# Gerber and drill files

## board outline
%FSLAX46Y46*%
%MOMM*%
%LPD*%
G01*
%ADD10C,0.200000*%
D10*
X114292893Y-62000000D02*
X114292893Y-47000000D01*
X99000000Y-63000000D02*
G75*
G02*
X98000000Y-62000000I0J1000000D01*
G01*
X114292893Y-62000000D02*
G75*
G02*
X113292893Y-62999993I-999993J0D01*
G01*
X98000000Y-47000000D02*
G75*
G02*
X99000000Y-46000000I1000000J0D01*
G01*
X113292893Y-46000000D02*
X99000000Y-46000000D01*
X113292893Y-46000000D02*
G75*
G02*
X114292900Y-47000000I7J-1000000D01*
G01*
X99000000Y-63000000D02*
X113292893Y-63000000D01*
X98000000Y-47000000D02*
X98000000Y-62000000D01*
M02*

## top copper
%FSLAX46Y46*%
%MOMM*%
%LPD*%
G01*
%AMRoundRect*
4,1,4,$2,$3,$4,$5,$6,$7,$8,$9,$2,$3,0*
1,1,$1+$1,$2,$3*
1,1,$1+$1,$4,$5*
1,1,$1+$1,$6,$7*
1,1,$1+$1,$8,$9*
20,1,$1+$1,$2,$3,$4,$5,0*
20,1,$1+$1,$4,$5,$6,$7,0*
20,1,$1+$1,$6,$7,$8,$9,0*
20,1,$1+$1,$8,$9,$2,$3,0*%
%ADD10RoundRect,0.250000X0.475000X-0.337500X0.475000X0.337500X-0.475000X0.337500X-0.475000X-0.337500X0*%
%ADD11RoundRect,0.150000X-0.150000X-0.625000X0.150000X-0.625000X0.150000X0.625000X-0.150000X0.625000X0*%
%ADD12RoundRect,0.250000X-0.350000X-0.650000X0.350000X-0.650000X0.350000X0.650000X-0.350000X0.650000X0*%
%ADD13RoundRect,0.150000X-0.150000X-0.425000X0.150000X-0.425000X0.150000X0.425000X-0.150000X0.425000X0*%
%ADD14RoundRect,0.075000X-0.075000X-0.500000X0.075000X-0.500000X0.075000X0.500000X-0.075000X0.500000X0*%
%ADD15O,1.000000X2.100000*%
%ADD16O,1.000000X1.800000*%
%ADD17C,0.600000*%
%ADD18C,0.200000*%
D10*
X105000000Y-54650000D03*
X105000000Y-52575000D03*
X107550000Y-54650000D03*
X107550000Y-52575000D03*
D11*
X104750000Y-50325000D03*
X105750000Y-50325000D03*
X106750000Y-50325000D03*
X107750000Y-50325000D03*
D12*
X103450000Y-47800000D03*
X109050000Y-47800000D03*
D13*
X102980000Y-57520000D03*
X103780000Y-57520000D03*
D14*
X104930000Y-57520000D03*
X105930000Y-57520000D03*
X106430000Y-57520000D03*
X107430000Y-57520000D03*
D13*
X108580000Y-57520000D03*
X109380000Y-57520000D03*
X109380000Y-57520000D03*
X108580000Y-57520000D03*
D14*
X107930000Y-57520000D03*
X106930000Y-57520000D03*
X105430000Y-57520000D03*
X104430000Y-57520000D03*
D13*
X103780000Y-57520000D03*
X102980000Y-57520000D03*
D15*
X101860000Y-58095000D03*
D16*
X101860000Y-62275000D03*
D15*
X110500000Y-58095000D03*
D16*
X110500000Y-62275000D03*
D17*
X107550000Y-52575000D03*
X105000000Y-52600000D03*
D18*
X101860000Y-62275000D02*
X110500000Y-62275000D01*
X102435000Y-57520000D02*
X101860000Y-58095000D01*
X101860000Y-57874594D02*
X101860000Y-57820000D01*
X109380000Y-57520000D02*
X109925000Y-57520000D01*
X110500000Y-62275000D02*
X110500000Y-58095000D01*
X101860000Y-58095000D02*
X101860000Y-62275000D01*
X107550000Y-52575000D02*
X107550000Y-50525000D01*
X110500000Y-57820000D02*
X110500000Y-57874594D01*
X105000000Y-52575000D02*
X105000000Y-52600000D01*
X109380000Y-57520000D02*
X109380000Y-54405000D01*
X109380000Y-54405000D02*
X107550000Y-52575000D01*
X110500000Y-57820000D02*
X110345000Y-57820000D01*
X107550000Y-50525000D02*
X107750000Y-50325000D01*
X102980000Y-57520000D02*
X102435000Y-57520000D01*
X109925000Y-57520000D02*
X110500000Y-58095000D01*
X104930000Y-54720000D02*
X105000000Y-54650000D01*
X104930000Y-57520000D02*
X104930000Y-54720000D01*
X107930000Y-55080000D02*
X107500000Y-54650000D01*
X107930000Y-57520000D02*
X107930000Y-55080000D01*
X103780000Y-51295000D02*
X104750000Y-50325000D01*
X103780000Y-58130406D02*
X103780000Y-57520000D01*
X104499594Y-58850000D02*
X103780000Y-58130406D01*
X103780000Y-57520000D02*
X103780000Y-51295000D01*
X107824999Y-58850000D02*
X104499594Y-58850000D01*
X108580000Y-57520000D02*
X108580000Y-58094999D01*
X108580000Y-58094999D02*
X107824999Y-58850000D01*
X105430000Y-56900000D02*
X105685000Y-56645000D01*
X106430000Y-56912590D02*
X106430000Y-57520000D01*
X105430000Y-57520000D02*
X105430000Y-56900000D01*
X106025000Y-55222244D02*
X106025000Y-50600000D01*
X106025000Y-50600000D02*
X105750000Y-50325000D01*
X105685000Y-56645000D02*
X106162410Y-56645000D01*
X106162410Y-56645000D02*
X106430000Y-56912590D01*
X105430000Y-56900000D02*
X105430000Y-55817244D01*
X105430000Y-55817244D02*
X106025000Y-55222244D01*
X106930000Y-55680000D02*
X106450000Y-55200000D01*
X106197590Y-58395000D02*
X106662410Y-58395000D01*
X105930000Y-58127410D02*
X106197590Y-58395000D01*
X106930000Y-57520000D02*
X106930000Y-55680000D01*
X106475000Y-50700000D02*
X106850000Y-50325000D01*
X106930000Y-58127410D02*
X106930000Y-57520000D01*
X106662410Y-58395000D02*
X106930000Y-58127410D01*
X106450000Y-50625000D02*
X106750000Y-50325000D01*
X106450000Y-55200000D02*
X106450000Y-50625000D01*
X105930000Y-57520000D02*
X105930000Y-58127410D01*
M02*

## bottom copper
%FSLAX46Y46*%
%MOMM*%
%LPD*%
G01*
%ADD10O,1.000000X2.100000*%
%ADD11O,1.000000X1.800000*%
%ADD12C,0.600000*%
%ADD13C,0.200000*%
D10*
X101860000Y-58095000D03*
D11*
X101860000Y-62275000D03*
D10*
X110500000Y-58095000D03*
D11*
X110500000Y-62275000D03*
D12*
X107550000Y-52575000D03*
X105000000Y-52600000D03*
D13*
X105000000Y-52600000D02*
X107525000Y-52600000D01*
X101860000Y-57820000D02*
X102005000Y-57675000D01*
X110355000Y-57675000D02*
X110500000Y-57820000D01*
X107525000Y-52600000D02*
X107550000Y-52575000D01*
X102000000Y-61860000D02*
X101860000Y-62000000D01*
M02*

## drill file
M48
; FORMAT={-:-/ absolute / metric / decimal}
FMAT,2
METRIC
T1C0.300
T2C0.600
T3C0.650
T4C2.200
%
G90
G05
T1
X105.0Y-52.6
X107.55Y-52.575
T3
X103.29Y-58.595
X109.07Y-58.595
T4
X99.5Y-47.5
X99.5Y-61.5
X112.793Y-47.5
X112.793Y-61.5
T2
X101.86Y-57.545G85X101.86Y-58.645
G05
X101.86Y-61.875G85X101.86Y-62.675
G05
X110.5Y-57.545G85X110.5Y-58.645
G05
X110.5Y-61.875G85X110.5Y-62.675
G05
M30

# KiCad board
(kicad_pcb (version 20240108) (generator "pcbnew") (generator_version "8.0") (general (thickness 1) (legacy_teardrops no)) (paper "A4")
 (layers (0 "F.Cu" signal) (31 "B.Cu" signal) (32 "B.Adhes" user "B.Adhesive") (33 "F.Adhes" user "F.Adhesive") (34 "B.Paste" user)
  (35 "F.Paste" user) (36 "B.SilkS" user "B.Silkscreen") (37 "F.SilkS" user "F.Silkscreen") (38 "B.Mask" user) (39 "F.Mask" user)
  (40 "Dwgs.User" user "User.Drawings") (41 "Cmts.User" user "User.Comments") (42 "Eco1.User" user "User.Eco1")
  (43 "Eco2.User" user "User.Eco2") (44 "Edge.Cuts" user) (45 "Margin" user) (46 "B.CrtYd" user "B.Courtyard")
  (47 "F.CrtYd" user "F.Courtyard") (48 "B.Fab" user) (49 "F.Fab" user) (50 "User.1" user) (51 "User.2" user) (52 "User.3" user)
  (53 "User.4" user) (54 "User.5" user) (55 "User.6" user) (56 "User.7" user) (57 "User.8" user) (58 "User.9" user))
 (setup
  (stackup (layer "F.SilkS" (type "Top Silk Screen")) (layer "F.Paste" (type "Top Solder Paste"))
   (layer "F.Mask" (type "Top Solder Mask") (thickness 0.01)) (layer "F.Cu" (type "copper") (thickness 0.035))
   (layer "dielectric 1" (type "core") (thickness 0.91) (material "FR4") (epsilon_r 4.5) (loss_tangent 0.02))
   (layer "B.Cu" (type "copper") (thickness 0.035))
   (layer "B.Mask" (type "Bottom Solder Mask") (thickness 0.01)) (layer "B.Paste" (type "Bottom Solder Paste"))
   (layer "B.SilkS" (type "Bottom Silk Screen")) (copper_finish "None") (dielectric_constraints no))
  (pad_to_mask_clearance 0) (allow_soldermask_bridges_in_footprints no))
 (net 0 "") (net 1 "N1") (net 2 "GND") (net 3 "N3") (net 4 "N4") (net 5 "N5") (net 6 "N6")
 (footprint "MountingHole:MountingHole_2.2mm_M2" (layer "F.Cu") (at 112.792893 47.5)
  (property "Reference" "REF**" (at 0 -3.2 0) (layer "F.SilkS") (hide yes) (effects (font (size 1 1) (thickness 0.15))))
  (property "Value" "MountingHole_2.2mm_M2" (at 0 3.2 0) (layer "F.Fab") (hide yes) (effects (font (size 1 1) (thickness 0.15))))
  (pad "" np_thru_hole circle (at 0 0) (size 2.2 2.2) (drill 2.2) (layers "*.Cu" "*.Mask")))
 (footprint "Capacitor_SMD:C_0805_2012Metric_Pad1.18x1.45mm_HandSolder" (layer "F.Cu") (at 105 53.6125 90)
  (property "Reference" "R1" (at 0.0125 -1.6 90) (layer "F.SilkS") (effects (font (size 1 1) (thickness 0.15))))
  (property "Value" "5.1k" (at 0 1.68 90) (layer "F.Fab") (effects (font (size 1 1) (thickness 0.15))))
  (pad "1" smd roundrect (at -1.0375 0 90) (size 1.175 1.45) (layers "F.Cu" "F.Paste" "F.Mask") (roundrect_rratio 0.212766) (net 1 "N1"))
  (pad "2" smd roundrect (at 1.0375 0 90) (size 1.175 1.45) (layers "F.Cu" "F.Paste" "F.Mask") (roundrect_rratio 0.212766) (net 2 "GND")))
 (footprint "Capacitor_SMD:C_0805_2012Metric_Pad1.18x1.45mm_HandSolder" (layer "F.Cu") (at 107.55 53.6125 90)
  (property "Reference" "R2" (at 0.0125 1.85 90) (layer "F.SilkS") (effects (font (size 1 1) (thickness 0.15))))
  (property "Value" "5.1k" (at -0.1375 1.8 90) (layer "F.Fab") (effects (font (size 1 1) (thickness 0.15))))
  (pad "1" smd roundrect (at -1.0375 0 90) (size 1.175 1.45) (layers "F.Cu" "F.Paste" "F.Mask") (roundrect_rratio 0.212766) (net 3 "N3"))
  (pad "2" smd roundrect (at 1.0375 0 90) (size 1.175 1.45) (layers "F.Cu" "F.Paste" "F.Mask") (roundrect_rratio 0.212766) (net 2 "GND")))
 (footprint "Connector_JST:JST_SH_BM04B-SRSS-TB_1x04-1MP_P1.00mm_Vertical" (layer "F.Cu") (at 106.25 49)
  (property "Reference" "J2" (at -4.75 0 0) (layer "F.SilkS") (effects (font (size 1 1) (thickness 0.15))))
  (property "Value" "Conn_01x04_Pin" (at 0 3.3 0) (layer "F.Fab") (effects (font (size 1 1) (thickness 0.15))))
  (pad "1" smd roundrect (at -1.5 1.325) (size 0.6 1.55) (layers "F.Cu" "F.Paste" "F.Mask") (roundrect_rratio 0.25) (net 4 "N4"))
  (pad "2" smd roundrect (at -0.5 1.325) (size 0.6 1.55) (layers "F.Cu" "F.Paste" "F.Mask") (roundrect_rratio 0.25) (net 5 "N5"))
  (pad "3" smd roundrect (at 0.5 1.325) (size 0.6 1.55) (layers "F.Cu" "F.Paste" "F.Mask") (roundrect_rratio 0.25) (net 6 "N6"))
  (pad "4" smd roundrect (at 1.5 1.325) (size 0.6 1.55) (layers "F.Cu" "F.Paste" "F.Mask") (roundrect_rratio 0.25) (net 2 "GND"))
  (pad "MP" smd roundrect (at -2.8 -1.2) (size 1.2 1.8) (layers "F.Cu" "F.Paste" "F.Mask") (roundrect_rratio 0.208333))
  (pad "MP" smd roundrect (at 2.8 -1.2) (size 1.2 1.8) (layers "F.Cu" "F.Paste" "F.Mask") (roundrect_rratio 0.208333)))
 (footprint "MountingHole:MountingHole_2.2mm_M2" (layer "F.Cu") (at 112.792893 61.5)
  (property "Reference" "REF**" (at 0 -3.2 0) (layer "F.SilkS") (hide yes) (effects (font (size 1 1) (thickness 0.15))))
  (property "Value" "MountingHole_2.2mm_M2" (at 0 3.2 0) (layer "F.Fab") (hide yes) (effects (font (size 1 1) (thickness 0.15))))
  (pad "" np_thru_hole circle (at 0 0) (size 2.2 2.2) (drill 2.2) (layers "*.Cu" "*.Mask")))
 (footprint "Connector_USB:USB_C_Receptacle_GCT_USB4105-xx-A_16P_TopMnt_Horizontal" (layer "F.Cu") (at 106.18 61.2)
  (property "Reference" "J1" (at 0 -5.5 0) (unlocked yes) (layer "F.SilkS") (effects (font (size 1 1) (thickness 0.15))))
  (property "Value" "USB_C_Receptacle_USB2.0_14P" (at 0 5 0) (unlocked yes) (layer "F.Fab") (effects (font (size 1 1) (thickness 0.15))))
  (pad "" np_thru_hole circle (at -2.89 -2.605) (size 0.65 0.65) (drill 0.65) (layers "F&B.Cu" "*.Mask"))
  (pad "" np_thru_hole circle (at 2.89 -2.605) (size 0.65 0.65) (drill 0.65) (layers "F&B.Cu" "*.Mask"))
  (pad "A1" smd roundrect (at -3.2 -3.68) (size 0.6 1.15) (layers "F.Cu" "F.Paste" "F.Mask") (roundrect_rratio 0.25) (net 2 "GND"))
  (pad "A4" smd roundrect (at -2.4 -3.68) (size 0.6 1.15) (layers "F.Cu" "F.Paste" "F.Mask") (roundrect_rratio 0.25) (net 4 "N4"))
  (pad "A5" smd roundrect (at -1.25 -3.68) (size 0.3 1.15) (layers "F.Cu" "F.Paste" "F.Mask") (roundrect_rratio 0.25) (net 1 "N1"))
  (pad "A6" smd roundrect (at -0.25 -3.68) (size 0.3 1.15) (layers "F.Cu" "F.Paste" "F.Mask") (roundrect_rratio 0.25) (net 6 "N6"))
  (pad "A7" smd roundrect (at 0.25 -3.68) (size 0.3 1.15) (layers "F.Cu" "F.Paste" "F.Mask") (roundrect_rratio 0.25) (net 5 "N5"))
  (pad "A8" smd roundrect (at 1.25 -3.68) (size 0.3 1.15) (layers "F.Cu" "F.Paste" "F.Mask") (roundrect_rratio 0.25))
  (pad "A9" smd roundrect (at 2.4 -3.68) (size 0.6 1.15) (layers "F.Cu" "F.Paste" "F.Mask") (roundrect_rratio 0.25) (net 4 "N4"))
  (pad "A12" smd roundrect (at 3.2 -3.68) (size 0.6 1.15) (layers "F.Cu" "F.Paste" "F.Mask") (roundrect_rratio 0.25) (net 2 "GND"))
  (pad "B1" smd roundrect (at 3.2 -3.68) (size 0.6 1.15) (layers "F.Cu" "F.Paste" "F.Mask") (roundrect_rratio 0.25) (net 2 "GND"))
  (pad "B4" smd roundrect (at 2.4 -3.68) (size 0.6 1.15) (layers "F.Cu" "F.Paste" "F.Mask") (roundrect_rratio 0.25) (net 4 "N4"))
  (pad "B5" smd roundrect (at 1.75 -3.68) (size 0.3 1.15) (layers "F.Cu" "F.Paste" "F.Mask") (roundrect_rratio 0.25) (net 3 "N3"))
  (pad "B6" smd roundrect (at 0.75 -3.68) (size 0.3 1.15) (layers "F.Cu" "F.Paste" "F.Mask") (roundrect_rratio 0.25) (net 6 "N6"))
  (pad "B7" smd roundrect (at -0.75 -3.68) (size 0.3 1.15) (layers "F.Cu" "F.Paste" "F.Mask") (roundrect_rratio 0.25) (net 5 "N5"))
  (pad "B8" smd roundrect (at -1.75 -3.68) (size 0.3 1.15) (layers "F.Cu" "F.Paste" "F.Mask") (roundrect_rratio 0.25))
  (pad "B9" smd roundrect (at -2.4 -3.68) (size 0.6 1.15) (layers "F.Cu" "F.Paste" "F.Mask") (roundrect_rratio 0.25) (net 4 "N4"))
  (pad "B12" smd roundrect (at -3.2 -3.68) (size 0.6 1.15) (layers "F.Cu" "F.Paste" "F.Mask") (roundrect_rratio 0.25) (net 2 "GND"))
  (pad "S1" thru_hole oval (at -4.32 -3.105) (size 1 2.1) (drill oval 0.6 1.7) (layers "*.Cu" "*.Mask" "F.Paste") (remove_unused_layers no)
   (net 2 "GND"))
  (pad "S1" thru_hole oval (at -4.32 1.075) (size 1 1.8) (drill oval 0.6 1.4) (layers "*.Cu" "*.Mask" "F.Paste") (remove_unused_layers no)
   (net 2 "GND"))
  (pad "S1" thru_hole oval (at 4.32 -3.105) (size 1 2.1) (drill oval 0.6 1.7) (layers "*.Cu" "*.Mask" "F.Paste") (remove_unused_layers no)
   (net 2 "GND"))
  (pad "S1" thru_hole oval (at 4.32 1.075) (size 1 1.8) (drill oval 0.6 1.4) (layers "*.Cu" "*.Mask" "F.Paste") (remove_unused_layers no)
   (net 2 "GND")))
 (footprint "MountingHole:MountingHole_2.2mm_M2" (layer "F.Cu") (at 99.5 61.5)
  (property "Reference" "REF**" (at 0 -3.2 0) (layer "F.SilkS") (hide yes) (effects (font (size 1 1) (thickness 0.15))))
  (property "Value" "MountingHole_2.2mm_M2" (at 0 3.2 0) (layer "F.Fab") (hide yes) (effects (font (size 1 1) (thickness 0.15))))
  (pad "" np_thru_hole circle (at 0 0) (size 2.2 2.2) (drill 2.2) (layers "*.Cu" "*.Mask")))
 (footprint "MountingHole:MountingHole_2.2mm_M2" (layer "F.Cu") (at 99.5 47.5)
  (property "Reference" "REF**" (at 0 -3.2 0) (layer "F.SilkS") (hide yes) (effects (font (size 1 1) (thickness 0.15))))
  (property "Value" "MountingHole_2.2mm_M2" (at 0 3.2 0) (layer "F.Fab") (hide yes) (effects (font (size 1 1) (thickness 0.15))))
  (pad "" np_thru_hole circle (at 0 0) (size 2.2 2.2) (drill 2.2) (layers "*.Cu" "*.Mask")))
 (gr_line (start 114.292893 62) (end 114.292893 47) (stroke (width 0.2) (type default)) (layer "Edge.Cuts"))
 (gr_arc (start 99 63) (mid 98.292896 62.707106) (end 98 62) (stroke (width 0.2) (type default)) (layer "Edge.Cuts"))
 (gr_arc (start 114.292893 62) (mid 114 62.707107) (end 113.292893 63) (stroke (width 0.2) (type default)) (layer "Edge.Cuts"))
 (gr_arc (start 98 47) (mid 98.292893 46.292893) (end 99 46) (stroke (width 0.2) (type default)) (layer "Edge.Cuts"))
 (gr_line (start 113.292893 46) (end 99 46) (stroke (width 0.2) (type default)) (layer "Edge.Cuts"))
 (gr_arc (start 113.292893 46) (mid 114 46.292893) (end 114.292893 47) (stroke (width 0.2) (type default)) (layer "Edge.Cuts"))
 (gr_line (start 99 63) (end 113.292893 63) (stroke (width 0.2) (type default)) (layer "Edge.Cuts"))
 (gr_line (start 98 47) (end 98 62) (stroke (width 0.2) (type default)) (layer "Edge.Cuts"))
 (segment (start 101.86 62.275) (end 110.5 62.275) (width 0.2) (layer "F.Cu") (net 2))
 (segment (start 102.435 57.52) (end 101.86 58.095) (width 0.2) (layer "F.Cu") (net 2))
 (segment (start 101.86 57.874594) (end 101.86 57.82) (width 0.2) (layer "F.Cu") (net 2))
 (segment (start 109.38 57.52) (end 109.925 57.52) (width 0.2) (layer "F.Cu") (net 2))
 (segment (start 110.5 62.275) (end 110.5 58.095) (width 0.2) (layer "F.Cu") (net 2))
 (segment (start 101.86 58.095) (end 101.86 62.275) (width 0.2) (layer "F.Cu") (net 2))
 (segment (start 107.55 52.575) (end 107.55 50.525) (width 0.2) (layer "F.Cu") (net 2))
 (segment (start 110.5 57.82) (end 110.5 57.874594) (width 0.2) (layer "F.Cu") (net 2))
 (segment (start 105 52.575) (end 105 52.6) (width 0.2) (layer "F.Cu") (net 2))
 (segment (start 109.38 57.52) (end 109.38 54.405) (width 0.2) (layer "F.Cu") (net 2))
 (segment (start 109.38 54.405) (end 107.55 52.575) (width 0.2) (layer "F.Cu") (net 2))
 (segment (start 110.5 57.82) (end 110.345 57.82) (width 0.2) (layer "F.Cu") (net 2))
 (segment (start 107.55 50.525) (end 107.75 50.325) (width 0.2) (layer "F.Cu") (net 2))
 (segment (start 102.98 57.52) (end 102.435 57.52) (width 0.2) (layer "F.Cu") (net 2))
 (segment (start 109.925 57.52) (end 110.5 58.095) (width 0.2) (layer "F.Cu") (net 2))
 (via (at 107.55 52.575) (size 0.6) (drill 0.3) (layers "F.Cu" "B.Cu") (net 2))
 (via (at 105 52.6) (size 0.6) (drill 0.3) (layers "F.Cu" "B.Cu") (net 2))
 (segment (start 105 52.6) (end 107.525 52.6) (width 0.2) (layer "B.Cu") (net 2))
 (segment (start 101.86 57.82) (end 102.005 57.675) (width 0.2) (layer "B.Cu") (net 2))
 (segment (start 110.355 57.675) (end 110.5 57.82) (width 0.2) (layer "B.Cu") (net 2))
 (segment (start 107.525 52.6) (end 107.55 52.575) (width 0.2) (layer "B.Cu") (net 2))
 (segment (start 102 61.86) (end 101.86 62) (width 0.2) (layer "B.Cu") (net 2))
 (segment (start 104.93 54.72) (end 105 54.65) (width 0.2) (layer "F.Cu") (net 1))
 (segment (start 104.93 57.52) (end 104.93 54.72) (width 0.2) (layer "F.Cu") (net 1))
 (segment (start 107.93 55.08) (end 107.5 54.65) (width 0.2) (layer "F.Cu") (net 3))
 (segment (start 107.93 57.52) (end 107.93 55.08) (width 0.2) (layer "F.Cu") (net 3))
 (segment (start 103.78 51.295) (end 104.75 50.325) (width 0.2) (layer "F.Cu") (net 4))
 (segment (start 103.78 58.130406) (end 103.78 57.52) (width 0.2) (layer "F.Cu") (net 4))
 (segment (start 104.499594 58.85) (end 103.78 58.130406) (width 0.2) (layer "F.Cu") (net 4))
 (segment (start 103.78 57.52) (end 103.78 51.295) (width 0.2) (layer "F.Cu") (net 4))
 (segment (start 107.824999 58.85) (end 104.499594 58.85) (width 0.2) (layer "F.Cu") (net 4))
 (segment (start 108.58 57.52) (end 108.58 58.094999) (width 0.2) (layer "F.Cu") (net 4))
 (segment (start 108.58 58.094999) (end 107.824999 58.85) (width 0.2) (layer "F.Cu") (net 4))
 (segment (start 105.43 56.9) (end 105.685 56.645) (width 0.2) (layer "F.Cu") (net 5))
 (segment (start 106.43 56.91259) (end 106.43 57.52) (width 0.2) (layer "F.Cu") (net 5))
 (segment (start 105.43 57.52) (end 105.43 56.9) (width 0.2) (layer "F.Cu") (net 5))
 (segment (start 106.025 55.222244) (end 106.025 50.6) (width 0.2) (layer "F.Cu") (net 5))
 (segment (start 106.025 50.6) (end 105.75 50.325) (width 0.2) (layer "F.Cu") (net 5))
 (segment (start 105.685 56.645) (end 106.16241 56.645) (width 0.2) (layer "F.Cu") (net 5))
 (segment (start 106.16241 56.645) (end 106.43 56.91259) (width 0.2) (layer "F.Cu") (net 5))
 (segment (start 105.43 56.9) (end 105.43 55.817244) (width 0.2) (layer "F.Cu") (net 5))
 (segment (start 105.43 55.817244) (end 106.025 55.222244) (width 0.2) (layer "F.Cu") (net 5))
 (segment (start 106.93 55.68) (end 106.45 55.2) (width 0.2) (layer "F.Cu") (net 6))
 (segment (start 106.19759 58.395) (end 106.66241 58.395) (width 0.2) (layer "F.Cu") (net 6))
 (segment (start 105.93 58.12741) (end 106.19759 58.395) (width 0.2) (layer "F.Cu") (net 6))
 (segment (start 106.93 57.52) (end 106.93 55.68) (width 0.2) (layer "F.Cu") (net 6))
 (segment (start 106.475 50.7) (end 106.85 50.325) (width 0.2) (layer "F.Cu") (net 6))
 (segment (start 106.93 58.12741) (end 106.93 57.52) (width 0.2) (layer "F.Cu") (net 6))
 (segment (start 106.66241 58.395) (end 106.93 58.12741) (width 0.2) (layer "F.Cu") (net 6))
 (segment (start 106.45 50.625) (end 106.75 50.325) (width 0.2) (layer "F.Cu") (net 6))
 (segment (start 106.45 55.2) (end 106.45 50.625) (width 0.2) (layer "F.Cu") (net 6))
 (segment (start 105.93 57.52) (end 105.93 58.12741) (width 0.2) (layer "F.Cu") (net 6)))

